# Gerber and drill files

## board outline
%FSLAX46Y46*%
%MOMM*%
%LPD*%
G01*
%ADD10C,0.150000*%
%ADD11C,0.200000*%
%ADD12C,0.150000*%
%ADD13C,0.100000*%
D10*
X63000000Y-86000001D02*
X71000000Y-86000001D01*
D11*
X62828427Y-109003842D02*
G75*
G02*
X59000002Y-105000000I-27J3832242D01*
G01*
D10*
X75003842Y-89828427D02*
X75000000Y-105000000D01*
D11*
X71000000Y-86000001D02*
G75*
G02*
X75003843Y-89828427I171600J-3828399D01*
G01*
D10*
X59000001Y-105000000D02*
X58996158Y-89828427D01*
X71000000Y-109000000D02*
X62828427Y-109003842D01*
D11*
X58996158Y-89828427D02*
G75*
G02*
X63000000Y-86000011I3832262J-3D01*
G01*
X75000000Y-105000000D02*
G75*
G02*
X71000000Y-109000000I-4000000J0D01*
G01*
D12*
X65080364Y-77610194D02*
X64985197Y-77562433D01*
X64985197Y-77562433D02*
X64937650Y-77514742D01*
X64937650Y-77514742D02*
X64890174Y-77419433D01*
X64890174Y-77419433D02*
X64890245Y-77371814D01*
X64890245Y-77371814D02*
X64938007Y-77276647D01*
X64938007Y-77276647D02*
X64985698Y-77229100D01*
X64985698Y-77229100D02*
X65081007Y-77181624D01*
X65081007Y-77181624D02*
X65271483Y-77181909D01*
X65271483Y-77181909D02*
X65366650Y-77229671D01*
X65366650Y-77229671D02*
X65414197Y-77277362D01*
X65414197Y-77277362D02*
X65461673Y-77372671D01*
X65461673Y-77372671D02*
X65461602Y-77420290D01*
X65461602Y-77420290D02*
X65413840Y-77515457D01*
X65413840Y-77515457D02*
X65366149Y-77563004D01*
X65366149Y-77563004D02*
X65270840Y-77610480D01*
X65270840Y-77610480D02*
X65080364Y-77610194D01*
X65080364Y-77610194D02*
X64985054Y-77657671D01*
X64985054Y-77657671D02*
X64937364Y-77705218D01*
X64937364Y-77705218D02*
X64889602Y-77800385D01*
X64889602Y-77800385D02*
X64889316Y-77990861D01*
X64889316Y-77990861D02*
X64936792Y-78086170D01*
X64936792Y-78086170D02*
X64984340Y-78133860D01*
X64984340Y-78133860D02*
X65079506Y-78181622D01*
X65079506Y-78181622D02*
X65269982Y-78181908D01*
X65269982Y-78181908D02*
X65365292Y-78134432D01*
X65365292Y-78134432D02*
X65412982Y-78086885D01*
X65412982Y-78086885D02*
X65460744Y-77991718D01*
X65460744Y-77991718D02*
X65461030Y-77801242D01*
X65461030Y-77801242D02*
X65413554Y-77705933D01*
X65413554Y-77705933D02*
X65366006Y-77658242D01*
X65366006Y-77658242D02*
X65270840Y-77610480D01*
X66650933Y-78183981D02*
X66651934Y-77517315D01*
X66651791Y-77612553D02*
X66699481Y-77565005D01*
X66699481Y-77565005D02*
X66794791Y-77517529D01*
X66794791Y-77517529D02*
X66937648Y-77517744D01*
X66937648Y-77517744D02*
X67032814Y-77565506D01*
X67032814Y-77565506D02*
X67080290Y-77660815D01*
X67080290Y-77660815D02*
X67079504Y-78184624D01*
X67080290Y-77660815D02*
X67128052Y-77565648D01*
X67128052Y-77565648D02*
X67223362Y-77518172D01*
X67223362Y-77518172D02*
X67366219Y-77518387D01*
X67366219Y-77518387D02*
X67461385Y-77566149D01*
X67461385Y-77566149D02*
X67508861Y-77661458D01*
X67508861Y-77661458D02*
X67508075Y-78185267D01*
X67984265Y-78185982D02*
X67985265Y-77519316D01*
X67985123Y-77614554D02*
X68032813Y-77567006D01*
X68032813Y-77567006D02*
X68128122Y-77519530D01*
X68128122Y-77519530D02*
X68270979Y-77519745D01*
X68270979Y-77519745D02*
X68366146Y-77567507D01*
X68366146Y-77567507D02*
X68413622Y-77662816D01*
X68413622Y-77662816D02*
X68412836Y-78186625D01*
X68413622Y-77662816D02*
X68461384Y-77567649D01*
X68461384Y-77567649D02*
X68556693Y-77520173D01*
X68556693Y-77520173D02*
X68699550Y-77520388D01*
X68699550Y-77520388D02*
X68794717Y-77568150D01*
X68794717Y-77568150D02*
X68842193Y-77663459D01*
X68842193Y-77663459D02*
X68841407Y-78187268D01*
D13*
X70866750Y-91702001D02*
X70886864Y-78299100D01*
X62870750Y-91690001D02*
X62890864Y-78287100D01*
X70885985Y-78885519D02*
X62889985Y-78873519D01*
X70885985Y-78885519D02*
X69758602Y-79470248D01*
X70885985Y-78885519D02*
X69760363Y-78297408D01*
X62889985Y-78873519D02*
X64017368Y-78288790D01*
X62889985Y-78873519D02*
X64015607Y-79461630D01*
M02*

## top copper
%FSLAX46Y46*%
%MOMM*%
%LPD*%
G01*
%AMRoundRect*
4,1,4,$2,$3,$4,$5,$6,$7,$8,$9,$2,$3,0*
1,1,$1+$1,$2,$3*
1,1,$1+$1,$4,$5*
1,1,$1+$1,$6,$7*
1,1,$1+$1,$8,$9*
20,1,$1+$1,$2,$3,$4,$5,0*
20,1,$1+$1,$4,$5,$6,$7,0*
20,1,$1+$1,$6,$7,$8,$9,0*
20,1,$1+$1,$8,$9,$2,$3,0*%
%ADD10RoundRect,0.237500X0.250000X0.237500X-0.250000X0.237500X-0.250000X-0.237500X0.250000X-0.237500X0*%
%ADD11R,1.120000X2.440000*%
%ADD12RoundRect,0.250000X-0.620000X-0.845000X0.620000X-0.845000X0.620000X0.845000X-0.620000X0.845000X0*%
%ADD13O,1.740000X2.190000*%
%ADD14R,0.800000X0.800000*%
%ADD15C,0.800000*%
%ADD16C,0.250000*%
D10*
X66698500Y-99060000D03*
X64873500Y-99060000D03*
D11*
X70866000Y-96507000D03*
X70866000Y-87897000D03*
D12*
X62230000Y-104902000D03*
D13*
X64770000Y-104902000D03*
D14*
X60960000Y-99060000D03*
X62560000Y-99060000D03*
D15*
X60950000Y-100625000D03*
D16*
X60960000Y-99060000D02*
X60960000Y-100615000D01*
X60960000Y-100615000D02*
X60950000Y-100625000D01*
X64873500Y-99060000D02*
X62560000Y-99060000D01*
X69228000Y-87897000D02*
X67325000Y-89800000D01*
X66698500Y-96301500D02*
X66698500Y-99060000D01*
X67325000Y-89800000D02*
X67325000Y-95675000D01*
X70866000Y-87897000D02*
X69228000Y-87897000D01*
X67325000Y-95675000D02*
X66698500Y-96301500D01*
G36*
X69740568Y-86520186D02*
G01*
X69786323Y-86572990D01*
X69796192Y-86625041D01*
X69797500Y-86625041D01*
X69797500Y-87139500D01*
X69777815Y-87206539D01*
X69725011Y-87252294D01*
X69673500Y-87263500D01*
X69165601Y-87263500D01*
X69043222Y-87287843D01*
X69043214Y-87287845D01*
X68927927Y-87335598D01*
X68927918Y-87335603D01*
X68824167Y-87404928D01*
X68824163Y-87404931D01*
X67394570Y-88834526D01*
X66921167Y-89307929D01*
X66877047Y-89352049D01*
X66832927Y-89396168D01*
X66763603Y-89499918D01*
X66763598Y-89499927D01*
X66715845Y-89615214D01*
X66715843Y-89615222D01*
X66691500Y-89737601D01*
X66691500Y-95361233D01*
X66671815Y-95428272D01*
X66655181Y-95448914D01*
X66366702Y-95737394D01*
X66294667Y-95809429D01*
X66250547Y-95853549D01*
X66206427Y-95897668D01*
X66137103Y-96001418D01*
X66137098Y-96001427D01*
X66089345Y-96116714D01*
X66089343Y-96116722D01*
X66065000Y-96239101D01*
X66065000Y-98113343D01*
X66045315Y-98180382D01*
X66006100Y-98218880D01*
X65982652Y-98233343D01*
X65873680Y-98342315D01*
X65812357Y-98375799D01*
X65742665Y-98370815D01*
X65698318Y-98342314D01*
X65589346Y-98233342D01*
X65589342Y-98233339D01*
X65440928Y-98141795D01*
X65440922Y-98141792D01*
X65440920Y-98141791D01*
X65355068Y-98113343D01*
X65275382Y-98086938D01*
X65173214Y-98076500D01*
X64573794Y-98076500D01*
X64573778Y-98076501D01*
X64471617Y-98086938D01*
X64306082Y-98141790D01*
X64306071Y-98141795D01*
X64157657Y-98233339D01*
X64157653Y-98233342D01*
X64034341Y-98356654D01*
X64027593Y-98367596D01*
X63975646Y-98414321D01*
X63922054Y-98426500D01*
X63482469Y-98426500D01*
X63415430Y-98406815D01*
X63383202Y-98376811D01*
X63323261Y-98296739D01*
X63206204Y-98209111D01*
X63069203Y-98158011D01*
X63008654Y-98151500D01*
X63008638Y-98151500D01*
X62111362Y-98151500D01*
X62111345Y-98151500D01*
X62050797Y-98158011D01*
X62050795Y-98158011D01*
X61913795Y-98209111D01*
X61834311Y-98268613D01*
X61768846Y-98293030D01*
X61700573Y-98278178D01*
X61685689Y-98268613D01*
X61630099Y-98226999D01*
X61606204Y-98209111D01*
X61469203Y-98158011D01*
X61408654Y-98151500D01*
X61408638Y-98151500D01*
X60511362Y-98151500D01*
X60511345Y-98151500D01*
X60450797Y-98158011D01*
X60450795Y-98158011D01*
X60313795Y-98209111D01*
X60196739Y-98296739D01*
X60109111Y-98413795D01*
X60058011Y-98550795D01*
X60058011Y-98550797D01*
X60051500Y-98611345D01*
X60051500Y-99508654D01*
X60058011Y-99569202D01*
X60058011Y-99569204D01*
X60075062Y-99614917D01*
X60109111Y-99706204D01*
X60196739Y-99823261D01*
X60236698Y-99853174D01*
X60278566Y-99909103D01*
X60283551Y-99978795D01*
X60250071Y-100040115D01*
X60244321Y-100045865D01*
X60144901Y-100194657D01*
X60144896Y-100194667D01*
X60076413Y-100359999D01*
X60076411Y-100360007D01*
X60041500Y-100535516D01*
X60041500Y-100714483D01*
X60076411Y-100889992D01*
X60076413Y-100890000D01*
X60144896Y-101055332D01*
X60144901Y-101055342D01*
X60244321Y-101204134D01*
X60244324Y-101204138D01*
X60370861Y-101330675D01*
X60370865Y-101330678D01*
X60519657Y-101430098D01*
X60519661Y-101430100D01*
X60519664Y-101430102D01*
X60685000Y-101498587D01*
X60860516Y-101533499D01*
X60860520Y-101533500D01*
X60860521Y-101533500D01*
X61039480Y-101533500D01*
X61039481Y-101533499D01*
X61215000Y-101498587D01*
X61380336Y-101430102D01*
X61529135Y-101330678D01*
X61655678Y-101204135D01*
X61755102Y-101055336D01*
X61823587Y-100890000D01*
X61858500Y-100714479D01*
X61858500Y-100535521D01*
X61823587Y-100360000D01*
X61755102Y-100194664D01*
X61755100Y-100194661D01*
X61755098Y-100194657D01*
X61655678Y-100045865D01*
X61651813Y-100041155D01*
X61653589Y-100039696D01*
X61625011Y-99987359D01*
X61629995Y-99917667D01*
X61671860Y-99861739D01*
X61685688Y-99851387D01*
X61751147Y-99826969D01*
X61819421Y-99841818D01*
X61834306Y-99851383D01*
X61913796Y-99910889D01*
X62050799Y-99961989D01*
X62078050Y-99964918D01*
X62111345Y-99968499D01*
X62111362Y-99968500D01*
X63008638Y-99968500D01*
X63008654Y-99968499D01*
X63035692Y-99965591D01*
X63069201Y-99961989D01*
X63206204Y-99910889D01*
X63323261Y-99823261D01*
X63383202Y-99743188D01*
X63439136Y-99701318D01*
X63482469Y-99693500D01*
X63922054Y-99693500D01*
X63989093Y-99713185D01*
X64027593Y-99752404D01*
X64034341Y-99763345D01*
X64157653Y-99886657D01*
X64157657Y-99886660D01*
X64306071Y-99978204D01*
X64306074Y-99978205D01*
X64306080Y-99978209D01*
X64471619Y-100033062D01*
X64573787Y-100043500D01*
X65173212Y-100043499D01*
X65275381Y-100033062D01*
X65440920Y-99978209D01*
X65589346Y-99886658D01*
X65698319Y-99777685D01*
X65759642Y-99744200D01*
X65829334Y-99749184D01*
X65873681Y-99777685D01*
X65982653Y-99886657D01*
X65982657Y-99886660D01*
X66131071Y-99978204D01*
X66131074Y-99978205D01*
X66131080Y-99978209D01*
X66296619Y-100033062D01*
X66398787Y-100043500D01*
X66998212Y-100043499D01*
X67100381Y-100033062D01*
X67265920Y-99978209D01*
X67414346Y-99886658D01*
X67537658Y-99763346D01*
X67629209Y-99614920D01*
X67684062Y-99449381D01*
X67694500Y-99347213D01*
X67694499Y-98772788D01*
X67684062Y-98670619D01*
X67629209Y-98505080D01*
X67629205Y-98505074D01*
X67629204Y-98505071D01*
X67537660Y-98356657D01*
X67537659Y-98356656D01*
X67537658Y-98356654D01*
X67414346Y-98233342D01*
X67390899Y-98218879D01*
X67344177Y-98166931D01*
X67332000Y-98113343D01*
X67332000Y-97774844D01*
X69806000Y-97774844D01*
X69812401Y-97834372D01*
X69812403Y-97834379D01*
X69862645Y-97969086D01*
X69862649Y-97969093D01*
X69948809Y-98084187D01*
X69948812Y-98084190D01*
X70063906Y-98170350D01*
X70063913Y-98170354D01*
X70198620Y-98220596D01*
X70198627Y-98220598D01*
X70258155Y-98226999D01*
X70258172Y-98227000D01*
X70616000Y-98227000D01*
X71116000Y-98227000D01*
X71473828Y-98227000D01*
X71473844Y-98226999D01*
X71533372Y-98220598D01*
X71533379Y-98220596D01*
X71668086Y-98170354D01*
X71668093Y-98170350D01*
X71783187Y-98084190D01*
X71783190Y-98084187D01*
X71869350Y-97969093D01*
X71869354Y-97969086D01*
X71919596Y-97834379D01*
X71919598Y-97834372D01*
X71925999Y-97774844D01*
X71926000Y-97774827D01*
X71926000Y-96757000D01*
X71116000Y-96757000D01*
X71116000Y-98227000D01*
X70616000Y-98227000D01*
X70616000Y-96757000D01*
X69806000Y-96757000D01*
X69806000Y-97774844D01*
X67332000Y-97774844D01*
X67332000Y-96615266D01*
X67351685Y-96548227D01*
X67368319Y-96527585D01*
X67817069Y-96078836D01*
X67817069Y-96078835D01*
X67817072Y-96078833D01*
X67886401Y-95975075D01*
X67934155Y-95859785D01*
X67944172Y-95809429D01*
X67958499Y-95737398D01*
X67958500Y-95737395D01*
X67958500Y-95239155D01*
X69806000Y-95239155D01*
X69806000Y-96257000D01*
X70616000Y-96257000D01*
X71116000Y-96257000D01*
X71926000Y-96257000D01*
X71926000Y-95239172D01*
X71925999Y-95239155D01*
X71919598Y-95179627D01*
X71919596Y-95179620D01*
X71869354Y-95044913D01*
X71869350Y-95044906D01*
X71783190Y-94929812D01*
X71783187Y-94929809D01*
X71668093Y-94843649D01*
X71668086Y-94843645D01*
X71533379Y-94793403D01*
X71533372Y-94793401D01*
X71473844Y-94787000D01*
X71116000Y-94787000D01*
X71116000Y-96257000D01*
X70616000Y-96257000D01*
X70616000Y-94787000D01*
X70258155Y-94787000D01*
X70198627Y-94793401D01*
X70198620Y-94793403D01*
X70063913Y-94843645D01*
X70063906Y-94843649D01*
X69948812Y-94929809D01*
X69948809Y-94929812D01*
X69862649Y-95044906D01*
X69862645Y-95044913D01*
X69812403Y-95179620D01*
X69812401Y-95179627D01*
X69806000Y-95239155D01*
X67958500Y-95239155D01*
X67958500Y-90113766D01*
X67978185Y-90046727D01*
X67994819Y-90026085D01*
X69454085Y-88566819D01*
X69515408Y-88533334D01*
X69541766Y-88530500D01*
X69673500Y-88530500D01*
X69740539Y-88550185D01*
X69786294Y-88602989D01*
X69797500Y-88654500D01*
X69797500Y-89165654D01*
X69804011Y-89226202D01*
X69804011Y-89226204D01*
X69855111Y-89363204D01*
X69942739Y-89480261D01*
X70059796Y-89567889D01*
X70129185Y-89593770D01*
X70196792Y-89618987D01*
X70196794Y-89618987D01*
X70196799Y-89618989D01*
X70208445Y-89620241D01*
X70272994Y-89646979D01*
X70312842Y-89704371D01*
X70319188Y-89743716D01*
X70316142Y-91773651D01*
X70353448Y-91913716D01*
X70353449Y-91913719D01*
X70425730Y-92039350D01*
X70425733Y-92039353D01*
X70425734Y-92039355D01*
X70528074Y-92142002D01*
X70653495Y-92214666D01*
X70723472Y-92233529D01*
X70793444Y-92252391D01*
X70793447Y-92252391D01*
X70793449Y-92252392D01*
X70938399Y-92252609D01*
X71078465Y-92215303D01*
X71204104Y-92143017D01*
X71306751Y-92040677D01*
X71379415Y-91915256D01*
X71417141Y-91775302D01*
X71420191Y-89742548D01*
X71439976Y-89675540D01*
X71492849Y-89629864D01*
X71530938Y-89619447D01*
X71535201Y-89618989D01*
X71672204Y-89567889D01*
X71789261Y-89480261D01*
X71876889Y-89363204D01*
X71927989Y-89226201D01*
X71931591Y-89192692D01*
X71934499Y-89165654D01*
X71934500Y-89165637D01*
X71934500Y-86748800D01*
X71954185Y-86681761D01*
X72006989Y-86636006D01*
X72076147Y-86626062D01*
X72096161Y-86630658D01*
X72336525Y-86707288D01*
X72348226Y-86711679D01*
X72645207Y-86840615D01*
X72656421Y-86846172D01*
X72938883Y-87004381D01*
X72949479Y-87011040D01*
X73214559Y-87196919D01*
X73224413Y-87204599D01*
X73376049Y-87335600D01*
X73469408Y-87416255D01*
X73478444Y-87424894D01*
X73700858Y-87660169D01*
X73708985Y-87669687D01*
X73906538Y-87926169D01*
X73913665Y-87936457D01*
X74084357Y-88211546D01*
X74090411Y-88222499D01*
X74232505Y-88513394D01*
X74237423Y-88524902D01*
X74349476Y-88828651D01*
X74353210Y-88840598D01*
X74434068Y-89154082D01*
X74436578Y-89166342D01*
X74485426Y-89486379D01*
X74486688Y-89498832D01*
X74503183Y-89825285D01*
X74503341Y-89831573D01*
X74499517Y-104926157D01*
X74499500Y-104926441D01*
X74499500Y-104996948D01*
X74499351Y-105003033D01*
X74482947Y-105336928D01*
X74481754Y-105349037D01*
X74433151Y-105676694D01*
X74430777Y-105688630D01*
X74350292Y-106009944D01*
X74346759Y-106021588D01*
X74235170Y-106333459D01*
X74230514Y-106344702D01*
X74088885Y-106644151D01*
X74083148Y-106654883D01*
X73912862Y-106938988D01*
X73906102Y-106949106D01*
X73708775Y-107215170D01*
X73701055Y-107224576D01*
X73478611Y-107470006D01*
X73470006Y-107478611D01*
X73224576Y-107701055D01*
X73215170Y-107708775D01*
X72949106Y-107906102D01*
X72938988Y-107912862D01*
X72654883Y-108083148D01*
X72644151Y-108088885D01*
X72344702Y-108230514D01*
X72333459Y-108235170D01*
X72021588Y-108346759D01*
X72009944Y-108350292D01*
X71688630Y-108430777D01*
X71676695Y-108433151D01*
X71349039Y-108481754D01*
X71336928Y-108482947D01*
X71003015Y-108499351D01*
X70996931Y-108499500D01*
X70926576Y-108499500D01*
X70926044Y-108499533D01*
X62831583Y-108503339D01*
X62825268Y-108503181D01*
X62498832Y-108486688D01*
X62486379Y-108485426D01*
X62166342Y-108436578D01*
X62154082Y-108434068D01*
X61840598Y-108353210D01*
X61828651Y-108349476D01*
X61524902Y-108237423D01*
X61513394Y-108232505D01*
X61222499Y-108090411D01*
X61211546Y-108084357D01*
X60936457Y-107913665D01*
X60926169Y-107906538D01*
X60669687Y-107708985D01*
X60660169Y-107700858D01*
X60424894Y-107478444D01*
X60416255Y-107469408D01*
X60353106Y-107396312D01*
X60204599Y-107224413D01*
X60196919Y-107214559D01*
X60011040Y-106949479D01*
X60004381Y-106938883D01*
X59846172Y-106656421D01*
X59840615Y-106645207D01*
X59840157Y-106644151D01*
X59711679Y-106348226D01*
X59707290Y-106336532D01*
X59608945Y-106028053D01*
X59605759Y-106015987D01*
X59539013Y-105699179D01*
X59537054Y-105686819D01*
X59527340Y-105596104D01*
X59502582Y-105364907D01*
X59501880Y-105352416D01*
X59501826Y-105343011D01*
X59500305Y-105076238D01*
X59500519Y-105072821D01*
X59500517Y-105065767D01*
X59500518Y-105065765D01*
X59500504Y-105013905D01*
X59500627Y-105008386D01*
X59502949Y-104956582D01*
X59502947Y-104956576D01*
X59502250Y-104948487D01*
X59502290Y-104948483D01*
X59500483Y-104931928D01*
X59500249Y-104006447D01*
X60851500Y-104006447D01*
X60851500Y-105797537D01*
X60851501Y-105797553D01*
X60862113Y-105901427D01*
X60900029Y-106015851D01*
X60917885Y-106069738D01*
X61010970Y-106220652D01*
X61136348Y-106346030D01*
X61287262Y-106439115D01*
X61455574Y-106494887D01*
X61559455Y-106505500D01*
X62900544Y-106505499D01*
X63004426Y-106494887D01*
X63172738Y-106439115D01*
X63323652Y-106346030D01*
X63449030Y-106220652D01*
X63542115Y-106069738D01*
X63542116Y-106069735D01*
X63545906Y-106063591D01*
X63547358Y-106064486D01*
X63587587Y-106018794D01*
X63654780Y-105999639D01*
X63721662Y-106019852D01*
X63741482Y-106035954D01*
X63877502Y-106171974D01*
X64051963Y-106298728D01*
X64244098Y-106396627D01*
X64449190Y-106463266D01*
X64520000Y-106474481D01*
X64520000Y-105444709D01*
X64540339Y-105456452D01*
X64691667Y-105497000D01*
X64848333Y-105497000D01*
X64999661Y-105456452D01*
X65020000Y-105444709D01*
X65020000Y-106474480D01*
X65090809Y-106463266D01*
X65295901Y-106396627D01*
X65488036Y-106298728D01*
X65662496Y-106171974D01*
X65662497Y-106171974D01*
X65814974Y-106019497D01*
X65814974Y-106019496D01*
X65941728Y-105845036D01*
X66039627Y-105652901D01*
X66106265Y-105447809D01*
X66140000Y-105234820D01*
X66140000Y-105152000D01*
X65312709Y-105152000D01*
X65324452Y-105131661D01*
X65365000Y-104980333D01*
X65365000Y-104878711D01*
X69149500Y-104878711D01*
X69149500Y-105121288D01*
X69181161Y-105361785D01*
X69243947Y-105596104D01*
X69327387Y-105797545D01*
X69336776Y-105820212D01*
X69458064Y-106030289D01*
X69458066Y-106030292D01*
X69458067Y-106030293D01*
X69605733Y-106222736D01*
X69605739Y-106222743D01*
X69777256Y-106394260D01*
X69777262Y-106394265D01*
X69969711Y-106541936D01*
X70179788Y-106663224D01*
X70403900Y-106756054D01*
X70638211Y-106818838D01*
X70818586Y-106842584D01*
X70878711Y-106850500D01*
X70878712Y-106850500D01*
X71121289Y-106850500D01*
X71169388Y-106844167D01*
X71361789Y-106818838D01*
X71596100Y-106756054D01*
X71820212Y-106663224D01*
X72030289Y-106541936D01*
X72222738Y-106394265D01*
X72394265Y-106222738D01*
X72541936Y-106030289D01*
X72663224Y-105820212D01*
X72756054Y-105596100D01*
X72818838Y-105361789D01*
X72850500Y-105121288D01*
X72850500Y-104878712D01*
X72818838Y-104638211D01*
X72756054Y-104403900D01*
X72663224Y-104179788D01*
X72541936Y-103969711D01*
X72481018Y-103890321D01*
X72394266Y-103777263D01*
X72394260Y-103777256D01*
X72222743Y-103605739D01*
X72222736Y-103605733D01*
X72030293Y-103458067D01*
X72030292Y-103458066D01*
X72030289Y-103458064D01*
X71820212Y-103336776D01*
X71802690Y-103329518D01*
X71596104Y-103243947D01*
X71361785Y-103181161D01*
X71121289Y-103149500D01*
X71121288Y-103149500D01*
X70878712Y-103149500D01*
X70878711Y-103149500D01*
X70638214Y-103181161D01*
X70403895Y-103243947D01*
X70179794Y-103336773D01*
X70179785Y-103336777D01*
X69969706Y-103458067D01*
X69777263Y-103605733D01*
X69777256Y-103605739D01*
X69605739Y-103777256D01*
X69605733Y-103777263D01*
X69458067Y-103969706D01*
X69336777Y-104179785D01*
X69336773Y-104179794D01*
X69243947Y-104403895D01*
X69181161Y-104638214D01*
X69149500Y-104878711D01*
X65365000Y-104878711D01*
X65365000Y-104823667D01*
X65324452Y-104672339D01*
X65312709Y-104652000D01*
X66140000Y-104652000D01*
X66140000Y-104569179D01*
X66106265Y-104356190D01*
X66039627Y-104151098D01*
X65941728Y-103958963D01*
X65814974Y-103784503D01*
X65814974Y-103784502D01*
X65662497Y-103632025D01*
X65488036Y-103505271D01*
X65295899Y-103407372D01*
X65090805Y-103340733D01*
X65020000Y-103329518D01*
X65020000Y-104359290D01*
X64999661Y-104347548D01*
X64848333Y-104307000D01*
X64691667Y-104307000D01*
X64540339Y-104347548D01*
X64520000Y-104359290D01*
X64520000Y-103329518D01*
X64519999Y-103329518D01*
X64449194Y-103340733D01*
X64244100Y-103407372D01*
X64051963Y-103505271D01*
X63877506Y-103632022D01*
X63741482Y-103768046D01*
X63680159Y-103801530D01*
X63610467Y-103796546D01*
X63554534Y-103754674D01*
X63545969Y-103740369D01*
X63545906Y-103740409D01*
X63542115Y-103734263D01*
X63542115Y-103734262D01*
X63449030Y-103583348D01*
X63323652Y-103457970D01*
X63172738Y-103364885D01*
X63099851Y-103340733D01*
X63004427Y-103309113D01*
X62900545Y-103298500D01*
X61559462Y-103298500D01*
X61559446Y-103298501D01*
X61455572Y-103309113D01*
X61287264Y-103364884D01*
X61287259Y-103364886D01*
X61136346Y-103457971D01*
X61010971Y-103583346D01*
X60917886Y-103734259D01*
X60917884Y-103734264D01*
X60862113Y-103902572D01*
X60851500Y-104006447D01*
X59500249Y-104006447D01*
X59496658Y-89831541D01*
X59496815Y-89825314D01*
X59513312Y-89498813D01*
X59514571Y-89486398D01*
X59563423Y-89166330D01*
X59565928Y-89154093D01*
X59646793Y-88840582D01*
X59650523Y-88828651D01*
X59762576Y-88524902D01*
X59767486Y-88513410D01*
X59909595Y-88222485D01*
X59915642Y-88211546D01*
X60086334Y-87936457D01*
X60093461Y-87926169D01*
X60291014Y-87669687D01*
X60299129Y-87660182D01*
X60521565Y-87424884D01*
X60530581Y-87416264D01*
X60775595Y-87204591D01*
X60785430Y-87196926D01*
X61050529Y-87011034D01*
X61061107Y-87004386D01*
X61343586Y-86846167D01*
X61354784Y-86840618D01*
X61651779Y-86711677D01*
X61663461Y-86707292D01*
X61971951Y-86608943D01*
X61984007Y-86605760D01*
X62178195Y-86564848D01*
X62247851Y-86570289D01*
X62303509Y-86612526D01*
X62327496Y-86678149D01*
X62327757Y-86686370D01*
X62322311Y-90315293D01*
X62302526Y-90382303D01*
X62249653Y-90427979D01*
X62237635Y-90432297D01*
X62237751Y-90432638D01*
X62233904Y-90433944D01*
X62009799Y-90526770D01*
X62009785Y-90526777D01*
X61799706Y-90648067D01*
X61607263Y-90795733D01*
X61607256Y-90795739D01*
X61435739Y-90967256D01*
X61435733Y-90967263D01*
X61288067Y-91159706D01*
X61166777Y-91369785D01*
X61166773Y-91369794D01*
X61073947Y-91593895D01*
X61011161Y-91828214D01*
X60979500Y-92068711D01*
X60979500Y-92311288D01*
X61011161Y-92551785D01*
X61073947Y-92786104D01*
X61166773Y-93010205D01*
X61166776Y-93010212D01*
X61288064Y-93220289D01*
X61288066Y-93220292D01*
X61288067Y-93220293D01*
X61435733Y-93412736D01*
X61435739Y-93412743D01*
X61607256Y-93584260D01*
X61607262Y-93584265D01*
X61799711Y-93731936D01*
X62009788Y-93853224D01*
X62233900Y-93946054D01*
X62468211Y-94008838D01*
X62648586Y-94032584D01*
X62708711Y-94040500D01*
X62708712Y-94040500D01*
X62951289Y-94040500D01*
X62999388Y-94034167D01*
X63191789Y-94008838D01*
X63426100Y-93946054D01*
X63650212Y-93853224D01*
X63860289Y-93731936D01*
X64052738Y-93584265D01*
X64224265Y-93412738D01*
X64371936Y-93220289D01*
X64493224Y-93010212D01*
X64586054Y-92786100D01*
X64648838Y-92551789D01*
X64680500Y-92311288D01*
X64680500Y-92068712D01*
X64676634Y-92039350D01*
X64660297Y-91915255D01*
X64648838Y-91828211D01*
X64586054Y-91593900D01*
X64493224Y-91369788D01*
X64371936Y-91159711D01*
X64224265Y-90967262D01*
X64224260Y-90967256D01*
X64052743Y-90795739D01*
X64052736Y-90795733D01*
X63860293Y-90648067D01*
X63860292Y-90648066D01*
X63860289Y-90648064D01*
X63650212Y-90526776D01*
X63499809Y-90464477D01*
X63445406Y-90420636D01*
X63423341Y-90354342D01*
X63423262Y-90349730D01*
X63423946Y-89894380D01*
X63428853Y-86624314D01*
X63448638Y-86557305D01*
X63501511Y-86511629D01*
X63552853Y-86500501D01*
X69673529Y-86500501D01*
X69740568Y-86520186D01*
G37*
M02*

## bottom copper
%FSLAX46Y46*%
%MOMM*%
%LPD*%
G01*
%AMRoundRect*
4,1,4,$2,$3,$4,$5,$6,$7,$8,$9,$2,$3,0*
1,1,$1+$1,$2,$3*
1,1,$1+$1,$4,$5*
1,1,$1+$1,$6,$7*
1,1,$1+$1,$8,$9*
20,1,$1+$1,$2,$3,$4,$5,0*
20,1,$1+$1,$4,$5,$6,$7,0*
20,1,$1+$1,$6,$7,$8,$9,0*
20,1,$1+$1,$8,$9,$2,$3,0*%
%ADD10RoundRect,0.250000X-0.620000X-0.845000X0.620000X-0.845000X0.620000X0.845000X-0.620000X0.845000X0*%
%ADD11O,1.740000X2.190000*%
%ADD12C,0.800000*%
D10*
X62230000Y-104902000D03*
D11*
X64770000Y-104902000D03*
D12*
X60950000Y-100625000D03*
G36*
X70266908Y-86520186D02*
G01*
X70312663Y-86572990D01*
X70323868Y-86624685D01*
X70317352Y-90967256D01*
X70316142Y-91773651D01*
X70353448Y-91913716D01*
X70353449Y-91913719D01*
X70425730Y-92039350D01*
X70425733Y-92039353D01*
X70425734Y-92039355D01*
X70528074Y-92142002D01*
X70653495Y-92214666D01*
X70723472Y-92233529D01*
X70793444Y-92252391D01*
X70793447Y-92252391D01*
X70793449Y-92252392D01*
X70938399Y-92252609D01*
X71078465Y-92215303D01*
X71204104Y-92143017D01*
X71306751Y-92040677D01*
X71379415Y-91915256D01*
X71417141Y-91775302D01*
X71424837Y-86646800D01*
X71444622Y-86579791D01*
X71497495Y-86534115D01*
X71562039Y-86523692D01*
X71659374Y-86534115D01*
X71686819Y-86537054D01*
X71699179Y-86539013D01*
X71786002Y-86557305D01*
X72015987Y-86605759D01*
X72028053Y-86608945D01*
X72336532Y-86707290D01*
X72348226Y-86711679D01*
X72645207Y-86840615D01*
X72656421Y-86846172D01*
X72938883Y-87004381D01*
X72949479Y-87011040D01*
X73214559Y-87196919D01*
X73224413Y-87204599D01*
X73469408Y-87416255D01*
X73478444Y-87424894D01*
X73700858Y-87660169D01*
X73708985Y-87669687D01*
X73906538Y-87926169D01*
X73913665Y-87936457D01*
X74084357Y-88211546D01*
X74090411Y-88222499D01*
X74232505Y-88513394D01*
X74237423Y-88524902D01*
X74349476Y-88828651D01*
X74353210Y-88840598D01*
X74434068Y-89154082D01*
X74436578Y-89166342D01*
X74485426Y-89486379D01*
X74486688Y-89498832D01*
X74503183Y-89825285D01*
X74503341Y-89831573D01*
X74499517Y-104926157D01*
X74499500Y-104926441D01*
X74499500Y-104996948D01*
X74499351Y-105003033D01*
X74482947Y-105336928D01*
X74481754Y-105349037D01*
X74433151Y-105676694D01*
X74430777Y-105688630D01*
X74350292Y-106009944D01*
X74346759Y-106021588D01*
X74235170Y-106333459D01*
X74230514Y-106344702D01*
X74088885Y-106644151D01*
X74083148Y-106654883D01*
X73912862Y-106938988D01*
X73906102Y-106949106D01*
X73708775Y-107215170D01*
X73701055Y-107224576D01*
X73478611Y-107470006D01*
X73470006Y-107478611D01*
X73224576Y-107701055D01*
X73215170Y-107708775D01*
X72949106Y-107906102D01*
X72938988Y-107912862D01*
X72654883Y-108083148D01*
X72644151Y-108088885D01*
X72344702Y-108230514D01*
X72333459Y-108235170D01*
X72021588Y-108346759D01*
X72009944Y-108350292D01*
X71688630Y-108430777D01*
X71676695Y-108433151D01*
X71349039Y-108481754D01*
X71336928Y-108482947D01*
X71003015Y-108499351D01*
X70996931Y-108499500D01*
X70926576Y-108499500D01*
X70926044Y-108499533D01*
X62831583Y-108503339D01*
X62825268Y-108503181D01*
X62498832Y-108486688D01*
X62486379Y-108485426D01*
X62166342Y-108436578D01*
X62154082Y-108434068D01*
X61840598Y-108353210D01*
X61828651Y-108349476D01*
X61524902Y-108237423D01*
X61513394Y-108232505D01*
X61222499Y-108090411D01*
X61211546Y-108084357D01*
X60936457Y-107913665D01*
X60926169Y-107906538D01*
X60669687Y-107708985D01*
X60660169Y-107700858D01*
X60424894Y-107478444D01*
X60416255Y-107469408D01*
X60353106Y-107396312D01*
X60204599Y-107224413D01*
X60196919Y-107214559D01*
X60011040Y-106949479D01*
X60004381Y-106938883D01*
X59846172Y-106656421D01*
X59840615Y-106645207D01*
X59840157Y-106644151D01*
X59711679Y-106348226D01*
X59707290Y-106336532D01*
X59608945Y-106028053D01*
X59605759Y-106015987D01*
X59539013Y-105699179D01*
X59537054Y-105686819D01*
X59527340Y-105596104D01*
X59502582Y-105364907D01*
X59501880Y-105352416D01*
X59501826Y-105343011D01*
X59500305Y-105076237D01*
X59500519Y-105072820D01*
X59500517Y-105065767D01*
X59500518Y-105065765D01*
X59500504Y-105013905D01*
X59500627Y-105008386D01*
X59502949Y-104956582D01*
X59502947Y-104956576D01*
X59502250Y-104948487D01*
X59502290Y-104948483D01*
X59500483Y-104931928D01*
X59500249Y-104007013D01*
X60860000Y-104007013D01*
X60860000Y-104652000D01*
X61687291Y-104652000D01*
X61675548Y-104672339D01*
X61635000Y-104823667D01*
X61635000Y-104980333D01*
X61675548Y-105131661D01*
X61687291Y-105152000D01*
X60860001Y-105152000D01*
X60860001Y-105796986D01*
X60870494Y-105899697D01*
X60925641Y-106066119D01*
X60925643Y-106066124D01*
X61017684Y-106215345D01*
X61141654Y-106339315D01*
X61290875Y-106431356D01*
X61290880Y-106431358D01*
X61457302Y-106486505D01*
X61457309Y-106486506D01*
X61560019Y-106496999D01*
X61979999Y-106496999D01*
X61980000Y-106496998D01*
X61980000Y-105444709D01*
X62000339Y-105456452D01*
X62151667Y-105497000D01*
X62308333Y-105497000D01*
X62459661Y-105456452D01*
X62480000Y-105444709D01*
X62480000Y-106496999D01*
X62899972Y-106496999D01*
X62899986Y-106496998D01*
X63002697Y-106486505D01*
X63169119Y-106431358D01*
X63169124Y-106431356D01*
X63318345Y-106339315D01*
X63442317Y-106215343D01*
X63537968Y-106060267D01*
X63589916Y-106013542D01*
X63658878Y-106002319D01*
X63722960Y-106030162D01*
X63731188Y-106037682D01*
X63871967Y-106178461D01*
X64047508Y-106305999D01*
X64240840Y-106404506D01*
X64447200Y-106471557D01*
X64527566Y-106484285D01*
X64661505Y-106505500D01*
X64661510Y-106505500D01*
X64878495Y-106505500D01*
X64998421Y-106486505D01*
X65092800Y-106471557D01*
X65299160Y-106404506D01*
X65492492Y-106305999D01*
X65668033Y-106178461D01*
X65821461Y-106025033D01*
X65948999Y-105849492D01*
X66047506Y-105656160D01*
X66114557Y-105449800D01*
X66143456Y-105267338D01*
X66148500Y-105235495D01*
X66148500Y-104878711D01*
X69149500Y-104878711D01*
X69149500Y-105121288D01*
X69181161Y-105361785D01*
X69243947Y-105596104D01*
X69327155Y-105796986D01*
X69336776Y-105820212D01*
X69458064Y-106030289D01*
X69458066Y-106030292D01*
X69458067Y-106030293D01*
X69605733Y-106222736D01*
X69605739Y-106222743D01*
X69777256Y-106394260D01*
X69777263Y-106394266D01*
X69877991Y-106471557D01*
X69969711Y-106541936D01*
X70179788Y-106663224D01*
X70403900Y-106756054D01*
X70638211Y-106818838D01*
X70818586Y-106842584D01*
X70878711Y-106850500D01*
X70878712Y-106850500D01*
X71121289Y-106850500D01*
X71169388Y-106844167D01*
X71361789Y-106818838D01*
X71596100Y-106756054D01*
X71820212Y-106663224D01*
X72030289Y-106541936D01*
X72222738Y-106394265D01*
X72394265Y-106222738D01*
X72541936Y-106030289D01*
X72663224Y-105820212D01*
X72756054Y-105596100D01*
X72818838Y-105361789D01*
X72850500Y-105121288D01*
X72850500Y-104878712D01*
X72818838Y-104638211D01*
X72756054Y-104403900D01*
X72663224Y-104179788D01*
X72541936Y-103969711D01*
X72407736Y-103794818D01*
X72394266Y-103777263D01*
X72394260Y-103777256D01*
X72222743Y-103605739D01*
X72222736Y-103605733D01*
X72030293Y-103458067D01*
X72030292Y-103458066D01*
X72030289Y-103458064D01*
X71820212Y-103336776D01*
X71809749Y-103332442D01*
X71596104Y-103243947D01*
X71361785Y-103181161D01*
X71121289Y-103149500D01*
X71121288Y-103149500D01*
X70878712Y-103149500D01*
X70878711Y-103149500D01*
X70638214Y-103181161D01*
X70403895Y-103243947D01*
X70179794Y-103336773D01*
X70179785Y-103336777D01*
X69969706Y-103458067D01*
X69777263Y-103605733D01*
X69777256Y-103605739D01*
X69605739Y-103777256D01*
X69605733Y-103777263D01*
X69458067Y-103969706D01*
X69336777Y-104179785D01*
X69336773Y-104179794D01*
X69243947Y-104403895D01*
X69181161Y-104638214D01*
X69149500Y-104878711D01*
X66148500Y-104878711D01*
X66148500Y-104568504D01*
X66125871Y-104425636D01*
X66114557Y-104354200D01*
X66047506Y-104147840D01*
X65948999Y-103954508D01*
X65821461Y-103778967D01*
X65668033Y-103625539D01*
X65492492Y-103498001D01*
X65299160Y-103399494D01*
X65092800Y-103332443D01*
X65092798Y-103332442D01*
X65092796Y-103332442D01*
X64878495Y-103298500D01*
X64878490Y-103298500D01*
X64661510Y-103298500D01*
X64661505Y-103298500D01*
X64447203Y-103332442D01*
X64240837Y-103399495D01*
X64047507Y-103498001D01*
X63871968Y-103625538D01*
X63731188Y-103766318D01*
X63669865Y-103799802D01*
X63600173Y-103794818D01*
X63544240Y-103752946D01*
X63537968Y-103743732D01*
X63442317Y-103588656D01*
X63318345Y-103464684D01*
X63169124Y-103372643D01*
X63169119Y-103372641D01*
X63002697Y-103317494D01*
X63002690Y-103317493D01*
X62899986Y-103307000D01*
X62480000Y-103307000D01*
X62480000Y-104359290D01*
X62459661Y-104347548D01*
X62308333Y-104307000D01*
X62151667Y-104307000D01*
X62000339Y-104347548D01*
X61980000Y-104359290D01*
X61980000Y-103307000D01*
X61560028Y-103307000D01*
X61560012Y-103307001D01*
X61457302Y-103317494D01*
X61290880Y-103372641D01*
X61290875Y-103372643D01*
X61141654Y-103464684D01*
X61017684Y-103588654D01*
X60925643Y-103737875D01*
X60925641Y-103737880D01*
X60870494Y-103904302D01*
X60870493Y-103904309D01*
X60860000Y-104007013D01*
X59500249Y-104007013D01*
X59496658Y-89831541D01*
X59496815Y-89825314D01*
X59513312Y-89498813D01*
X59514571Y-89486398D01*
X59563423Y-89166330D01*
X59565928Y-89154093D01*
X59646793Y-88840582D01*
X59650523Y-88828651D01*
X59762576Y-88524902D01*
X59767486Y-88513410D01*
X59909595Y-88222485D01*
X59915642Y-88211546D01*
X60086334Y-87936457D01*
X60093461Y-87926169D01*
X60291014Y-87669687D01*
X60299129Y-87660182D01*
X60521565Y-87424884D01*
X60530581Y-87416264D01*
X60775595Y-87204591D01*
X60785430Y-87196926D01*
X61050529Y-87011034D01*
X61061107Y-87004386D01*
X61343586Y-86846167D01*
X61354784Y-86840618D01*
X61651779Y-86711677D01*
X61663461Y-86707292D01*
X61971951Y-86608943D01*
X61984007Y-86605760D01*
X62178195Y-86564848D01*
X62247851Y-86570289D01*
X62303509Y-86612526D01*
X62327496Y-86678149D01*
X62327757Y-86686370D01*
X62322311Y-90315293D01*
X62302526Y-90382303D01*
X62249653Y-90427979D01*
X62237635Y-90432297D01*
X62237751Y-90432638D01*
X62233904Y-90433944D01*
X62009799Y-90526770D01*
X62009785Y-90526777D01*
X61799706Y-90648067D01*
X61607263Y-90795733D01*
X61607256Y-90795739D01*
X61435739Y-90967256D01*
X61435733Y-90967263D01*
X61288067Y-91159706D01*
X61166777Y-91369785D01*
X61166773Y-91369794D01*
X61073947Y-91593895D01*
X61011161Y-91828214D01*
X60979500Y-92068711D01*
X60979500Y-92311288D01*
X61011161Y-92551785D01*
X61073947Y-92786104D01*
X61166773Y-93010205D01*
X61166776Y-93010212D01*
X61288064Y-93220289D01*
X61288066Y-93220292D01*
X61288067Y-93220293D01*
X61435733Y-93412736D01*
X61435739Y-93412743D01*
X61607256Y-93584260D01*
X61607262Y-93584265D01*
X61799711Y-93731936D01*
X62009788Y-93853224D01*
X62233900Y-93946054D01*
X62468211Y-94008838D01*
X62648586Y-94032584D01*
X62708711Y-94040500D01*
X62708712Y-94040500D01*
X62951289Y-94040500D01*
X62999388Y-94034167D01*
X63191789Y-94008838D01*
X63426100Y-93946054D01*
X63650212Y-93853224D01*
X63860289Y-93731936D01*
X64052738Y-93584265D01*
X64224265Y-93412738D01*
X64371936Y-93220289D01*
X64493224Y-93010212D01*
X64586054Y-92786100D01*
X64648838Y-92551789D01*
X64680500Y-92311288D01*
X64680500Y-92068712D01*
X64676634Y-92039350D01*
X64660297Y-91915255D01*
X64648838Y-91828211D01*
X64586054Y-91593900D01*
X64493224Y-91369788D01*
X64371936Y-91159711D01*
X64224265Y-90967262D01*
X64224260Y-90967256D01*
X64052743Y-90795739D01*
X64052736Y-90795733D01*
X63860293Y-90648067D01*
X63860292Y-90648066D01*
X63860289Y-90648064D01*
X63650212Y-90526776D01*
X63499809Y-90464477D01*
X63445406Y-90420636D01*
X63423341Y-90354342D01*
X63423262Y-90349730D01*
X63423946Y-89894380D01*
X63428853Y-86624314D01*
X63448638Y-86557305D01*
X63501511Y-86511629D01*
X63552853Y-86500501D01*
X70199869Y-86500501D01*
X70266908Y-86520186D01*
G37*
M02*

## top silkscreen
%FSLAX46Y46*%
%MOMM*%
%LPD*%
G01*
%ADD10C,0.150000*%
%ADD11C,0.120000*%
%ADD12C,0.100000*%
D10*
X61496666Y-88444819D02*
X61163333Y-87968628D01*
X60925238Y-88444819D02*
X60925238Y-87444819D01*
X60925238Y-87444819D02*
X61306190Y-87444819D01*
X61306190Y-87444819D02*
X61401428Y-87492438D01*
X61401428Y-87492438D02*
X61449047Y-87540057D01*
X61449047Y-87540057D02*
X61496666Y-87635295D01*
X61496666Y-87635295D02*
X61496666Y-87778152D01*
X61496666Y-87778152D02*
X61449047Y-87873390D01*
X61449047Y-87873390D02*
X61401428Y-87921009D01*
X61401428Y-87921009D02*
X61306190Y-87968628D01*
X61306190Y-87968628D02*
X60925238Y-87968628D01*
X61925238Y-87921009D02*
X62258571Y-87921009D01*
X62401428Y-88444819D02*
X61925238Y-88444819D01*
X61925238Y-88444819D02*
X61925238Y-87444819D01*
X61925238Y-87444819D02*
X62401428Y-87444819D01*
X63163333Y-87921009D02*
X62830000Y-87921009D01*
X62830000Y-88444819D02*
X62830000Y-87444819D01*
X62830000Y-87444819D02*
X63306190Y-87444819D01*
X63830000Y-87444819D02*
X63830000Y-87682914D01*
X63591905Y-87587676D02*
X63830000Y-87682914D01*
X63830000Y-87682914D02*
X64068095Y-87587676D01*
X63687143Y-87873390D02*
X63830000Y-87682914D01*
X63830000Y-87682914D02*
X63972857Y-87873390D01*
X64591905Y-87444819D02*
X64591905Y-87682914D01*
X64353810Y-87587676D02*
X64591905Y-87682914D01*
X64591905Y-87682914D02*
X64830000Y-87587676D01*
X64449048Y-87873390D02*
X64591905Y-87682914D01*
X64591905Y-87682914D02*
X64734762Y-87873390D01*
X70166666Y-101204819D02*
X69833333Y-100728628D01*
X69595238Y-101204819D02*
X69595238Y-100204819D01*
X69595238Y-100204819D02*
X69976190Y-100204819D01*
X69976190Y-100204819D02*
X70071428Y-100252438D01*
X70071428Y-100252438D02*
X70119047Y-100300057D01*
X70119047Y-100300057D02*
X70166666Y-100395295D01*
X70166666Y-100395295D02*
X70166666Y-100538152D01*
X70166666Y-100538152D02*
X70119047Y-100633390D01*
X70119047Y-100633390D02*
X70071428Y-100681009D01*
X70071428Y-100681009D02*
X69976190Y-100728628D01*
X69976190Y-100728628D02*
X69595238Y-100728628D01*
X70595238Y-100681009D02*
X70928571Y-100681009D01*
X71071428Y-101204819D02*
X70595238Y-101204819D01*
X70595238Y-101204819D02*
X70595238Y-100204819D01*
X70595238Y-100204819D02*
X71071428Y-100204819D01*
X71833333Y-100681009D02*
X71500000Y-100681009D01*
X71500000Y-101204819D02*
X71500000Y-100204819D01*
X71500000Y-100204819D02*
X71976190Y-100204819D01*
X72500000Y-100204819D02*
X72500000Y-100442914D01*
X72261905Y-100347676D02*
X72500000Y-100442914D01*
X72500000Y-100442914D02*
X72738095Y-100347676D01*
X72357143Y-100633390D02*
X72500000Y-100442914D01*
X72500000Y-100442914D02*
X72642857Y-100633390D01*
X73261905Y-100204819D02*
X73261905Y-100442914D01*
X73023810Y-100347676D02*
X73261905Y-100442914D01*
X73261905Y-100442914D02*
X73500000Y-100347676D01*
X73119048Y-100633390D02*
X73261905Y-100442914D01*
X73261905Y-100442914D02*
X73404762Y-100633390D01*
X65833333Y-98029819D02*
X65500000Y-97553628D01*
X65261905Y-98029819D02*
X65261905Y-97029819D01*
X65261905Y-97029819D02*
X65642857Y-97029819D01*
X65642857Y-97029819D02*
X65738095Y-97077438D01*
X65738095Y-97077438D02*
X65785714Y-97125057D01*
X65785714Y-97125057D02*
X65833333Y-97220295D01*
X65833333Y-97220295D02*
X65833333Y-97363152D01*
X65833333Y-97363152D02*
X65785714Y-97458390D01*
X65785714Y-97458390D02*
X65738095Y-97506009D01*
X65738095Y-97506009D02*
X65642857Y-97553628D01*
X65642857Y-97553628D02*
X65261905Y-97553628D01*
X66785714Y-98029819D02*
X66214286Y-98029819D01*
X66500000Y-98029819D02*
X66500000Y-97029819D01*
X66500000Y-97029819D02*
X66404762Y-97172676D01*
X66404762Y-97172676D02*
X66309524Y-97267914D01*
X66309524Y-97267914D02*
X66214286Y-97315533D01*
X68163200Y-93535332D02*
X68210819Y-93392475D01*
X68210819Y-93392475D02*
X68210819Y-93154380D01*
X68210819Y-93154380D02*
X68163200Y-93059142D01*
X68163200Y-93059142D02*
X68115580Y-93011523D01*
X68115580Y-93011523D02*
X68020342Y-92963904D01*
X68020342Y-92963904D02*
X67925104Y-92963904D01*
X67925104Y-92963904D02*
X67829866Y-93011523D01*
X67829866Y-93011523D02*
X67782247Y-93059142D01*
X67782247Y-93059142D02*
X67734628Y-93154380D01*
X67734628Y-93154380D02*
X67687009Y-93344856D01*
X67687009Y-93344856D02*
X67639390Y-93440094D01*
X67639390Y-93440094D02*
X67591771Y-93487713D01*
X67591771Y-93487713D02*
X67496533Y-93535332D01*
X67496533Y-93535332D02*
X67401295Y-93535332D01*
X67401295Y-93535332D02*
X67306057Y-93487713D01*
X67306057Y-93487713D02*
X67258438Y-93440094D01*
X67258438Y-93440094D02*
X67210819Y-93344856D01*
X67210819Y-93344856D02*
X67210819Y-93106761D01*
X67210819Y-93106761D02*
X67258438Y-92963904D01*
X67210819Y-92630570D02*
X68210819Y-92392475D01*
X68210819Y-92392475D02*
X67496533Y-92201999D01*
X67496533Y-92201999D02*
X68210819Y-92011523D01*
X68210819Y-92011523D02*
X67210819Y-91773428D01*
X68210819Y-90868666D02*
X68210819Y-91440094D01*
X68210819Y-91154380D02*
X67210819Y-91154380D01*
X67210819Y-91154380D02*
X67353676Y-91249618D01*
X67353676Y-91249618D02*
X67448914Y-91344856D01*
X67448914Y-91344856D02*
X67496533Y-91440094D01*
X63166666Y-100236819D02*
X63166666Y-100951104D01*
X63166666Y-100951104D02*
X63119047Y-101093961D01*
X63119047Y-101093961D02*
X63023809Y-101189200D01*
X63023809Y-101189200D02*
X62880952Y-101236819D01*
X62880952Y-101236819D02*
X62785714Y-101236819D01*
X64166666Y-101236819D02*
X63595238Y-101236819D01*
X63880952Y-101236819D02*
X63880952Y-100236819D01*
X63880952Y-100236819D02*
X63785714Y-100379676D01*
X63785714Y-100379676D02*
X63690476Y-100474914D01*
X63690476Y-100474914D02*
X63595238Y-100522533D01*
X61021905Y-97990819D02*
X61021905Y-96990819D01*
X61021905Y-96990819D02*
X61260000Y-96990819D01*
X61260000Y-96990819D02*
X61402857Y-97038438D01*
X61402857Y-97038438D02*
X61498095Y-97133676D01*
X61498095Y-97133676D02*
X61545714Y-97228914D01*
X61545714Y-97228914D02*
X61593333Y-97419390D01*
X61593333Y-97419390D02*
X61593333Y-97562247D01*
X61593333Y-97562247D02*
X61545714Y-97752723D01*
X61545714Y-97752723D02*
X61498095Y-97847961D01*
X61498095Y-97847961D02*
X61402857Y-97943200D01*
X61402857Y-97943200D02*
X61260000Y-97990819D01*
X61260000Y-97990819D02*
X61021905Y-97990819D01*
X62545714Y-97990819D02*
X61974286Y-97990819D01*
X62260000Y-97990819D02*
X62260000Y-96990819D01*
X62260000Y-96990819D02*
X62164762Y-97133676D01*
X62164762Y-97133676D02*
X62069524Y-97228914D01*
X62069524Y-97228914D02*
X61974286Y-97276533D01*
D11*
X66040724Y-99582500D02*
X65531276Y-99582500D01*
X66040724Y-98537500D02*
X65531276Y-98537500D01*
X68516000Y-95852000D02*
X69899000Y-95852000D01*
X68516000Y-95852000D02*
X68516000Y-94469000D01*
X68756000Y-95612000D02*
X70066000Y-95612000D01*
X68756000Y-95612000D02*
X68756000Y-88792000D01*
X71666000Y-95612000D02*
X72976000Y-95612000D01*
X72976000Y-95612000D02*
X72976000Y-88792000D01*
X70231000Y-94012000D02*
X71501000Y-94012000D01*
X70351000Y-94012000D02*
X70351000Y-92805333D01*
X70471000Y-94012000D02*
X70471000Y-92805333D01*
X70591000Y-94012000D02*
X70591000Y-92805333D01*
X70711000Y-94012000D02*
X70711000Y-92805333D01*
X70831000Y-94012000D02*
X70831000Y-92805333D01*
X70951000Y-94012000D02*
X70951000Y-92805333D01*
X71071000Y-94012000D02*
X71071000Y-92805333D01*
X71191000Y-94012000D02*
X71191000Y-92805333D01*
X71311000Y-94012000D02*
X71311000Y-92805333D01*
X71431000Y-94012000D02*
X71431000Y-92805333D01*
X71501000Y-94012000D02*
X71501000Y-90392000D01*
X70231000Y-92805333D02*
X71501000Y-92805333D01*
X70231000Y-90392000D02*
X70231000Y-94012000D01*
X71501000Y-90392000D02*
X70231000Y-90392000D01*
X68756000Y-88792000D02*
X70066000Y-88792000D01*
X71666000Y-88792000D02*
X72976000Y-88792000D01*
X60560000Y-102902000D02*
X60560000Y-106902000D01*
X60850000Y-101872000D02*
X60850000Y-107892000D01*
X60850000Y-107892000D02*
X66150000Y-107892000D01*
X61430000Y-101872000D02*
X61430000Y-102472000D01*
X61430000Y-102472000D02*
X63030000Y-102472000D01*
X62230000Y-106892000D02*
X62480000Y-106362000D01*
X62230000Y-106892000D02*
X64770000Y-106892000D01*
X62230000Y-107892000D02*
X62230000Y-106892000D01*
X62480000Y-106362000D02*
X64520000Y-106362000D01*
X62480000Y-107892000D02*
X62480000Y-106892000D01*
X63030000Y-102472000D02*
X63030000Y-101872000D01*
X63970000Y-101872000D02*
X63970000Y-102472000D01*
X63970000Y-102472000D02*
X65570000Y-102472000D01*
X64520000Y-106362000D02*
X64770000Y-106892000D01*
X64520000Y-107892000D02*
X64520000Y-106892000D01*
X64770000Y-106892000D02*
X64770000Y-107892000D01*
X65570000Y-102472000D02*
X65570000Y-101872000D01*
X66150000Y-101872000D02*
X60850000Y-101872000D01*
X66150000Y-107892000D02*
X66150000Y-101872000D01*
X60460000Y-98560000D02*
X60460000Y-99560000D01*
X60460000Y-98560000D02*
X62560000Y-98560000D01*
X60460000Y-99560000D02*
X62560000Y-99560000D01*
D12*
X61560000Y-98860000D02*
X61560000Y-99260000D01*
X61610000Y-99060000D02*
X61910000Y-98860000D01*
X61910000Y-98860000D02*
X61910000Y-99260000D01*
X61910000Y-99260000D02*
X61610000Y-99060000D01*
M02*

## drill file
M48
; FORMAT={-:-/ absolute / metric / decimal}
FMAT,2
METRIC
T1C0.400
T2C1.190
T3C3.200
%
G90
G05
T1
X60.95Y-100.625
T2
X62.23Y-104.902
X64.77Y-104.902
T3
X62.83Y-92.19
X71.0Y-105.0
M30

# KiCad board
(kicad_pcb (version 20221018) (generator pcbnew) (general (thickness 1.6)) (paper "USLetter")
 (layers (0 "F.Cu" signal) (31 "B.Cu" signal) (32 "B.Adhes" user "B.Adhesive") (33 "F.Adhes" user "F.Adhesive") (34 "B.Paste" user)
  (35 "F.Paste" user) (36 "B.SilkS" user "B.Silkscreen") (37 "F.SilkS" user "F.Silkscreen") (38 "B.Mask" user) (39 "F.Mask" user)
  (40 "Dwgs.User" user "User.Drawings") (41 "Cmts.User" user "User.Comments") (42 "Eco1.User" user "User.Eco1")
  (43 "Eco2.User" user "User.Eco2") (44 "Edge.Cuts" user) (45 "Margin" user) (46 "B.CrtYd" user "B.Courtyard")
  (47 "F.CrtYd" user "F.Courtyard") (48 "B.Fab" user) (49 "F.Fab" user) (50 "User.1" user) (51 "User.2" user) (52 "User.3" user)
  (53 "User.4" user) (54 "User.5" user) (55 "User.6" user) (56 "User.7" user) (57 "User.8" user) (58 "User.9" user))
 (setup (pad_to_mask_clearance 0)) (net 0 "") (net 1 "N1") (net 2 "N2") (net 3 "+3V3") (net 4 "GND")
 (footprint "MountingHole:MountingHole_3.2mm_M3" (layer "F.Cu") (at 62.83 92.19)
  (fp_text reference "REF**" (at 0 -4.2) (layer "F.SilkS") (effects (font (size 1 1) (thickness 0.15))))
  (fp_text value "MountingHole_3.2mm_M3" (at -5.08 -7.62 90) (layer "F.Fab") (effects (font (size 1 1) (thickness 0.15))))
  (pad "" np_thru_hole circle (at 0 0) (size 3.2 3.2) (drill 3.2) (layers "*.Cu" "*.Mask")))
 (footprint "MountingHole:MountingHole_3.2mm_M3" (layer "F.Cu") (at 71 105)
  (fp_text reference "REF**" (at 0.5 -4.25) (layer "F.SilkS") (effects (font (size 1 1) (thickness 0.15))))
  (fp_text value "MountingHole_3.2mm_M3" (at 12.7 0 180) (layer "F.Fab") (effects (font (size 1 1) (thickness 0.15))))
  (pad "" np_thru_hole circle (at 0 0) (size 3.2 3.2) (drill 3.2) (layers "*.Cu" "*.Mask")))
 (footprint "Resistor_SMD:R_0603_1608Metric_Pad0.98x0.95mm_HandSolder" (layer "F.Cu") (at 65.786 99.06 180)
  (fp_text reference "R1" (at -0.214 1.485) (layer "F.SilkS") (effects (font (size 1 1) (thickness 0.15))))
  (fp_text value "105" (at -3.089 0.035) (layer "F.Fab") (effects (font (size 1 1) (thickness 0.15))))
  (fp_line (start -0.254724 -0.5225) (end 0.254724 -0.5225) (stroke (width 0.12) (type solid)) (layer "F.SilkS"))
  (fp_line (start -0.254724 0.5225) (end 0.254724 0.5225) (stroke (width 0.12) (type solid)) (layer "F.SilkS"))
  (pad "1" smd roundrect (at -0.9125 0 180) (size 0.975 0.95) (layers "F.Cu" "F.Paste" "F.Mask") (roundrect_rratio 0.25) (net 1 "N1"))
  (pad "2" smd roundrect (at 0.9125 0 180) (size 0.975 0.95) (layers "F.Cu" "F.Paste" "F.Mask") (roundrect_rratio 0.25) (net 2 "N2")))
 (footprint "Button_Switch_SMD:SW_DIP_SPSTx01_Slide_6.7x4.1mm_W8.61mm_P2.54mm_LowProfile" (layer "F.Cu") (at 70.866 92.202 90)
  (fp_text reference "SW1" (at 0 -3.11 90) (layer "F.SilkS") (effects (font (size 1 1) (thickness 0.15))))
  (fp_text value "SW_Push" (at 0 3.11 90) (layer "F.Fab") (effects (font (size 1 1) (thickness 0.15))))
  (fp_line (start -3.65 -2.35) (end -3.65 -0.967) (stroke (width 0.12) (type solid)) (layer "F.SilkS"))
  (fp_line (start -3.65 -2.35) (end -2.267 -2.35) (stroke (width 0.12) (type solid)) (layer "F.SilkS"))
  (fp_line (start -3.41 -2.11) (end -3.41 -0.8) (stroke (width 0.12) (type solid)) (layer "F.SilkS"))
  (fp_line (start -3.41 -2.11) (end 3.41 -2.11) (stroke (width 0.12) (type solid)) (layer "F.SilkS"))
  (fp_line (start -3.41 0.8) (end -3.41 2.11) (stroke (width 0.12) (type solid)) (layer "F.SilkS"))
  (fp_line (start -3.41 2.11) (end 3.41 2.11) (stroke (width 0.12) (type solid)) (layer "F.SilkS"))
  (fp_line (start -1.81 -0.635) (end -1.81 0.635) (stroke (width 0.12) (type solid)) (layer "F.SilkS"))
  (fp_line (start -1.81 -0.515) (end -0.603333 -0.515) (stroke (width 0.12) (type solid)) (layer "F.SilkS"))
  (fp_line (start -1.81 -0.395) (end -0.603333 -0.395) (stroke (width 0.12) (type solid)) (layer "F.SilkS"))
  (fp_line (start -1.81 -0.275) (end -0.603333 -0.275) (stroke (width 0.12) (type solid)) (layer "F.SilkS"))
  (fp_line (start -1.81 -0.155) (end -0.603333 -0.155) (stroke (width 0.12) (type solid)) (layer "F.SilkS"))
  (fp_line (start -1.81 -0.035) (end -0.603333 -0.035) (stroke (width 0.12) (type solid)) (layer "F.SilkS"))
  (fp_line (start -1.81 0.085) (end -0.603333 0.085) (stroke (width 0.12) (type solid)) (layer "F.SilkS"))
  (fp_line (start -1.81 0.205) (end -0.603333 0.205) (stroke (width 0.12) (type solid)) (layer "F.SilkS"))
  (fp_line (start -1.81 0.325) (end -0.603333 0.325) (stroke (width 0.12) (type solid)) (layer "F.SilkS"))
  (fp_line (start -1.81 0.445) (end -0.603333 0.445) (stroke (width 0.12) (type solid)) (layer "F.SilkS"))
  (fp_line (start -1.81 0.565) (end -0.603333 0.565) (stroke (width 0.12) (type solid)) (layer "F.SilkS"))
  (fp_line (start -1.81 0.635) (end 1.81 0.635) (stroke (width 0.12) (type solid)) (layer "F.SilkS"))
  (fp_line (start -0.603333 -0.635) (end -0.603333 0.635) (stroke (width 0.12) (type solid)) (layer "F.SilkS"))
  (fp_line (start 1.81 -0.635) (end -1.81 -0.635) (stroke (width 0.12) (type solid)) (layer "F.SilkS"))
  (fp_line (start 1.81 0.635) (end 1.81 -0.635) (stroke (width 0.12) (type solid)) (layer "F.SilkS"))
  (fp_line (start 3.41 -2.11) (end 3.41 -0.8) (stroke (width 0.12) (type solid)) (layer "F.SilkS"))
  (fp_line (start 3.41 0.8) (end 3.41 2.11) (stroke (width 0.12) (type solid)) (layer "F.SilkS"))
  (pad "1" smd rect (at -4.305 0 90) (size 2.44 1.12) (layers "F.Cu" "F.Paste" "F.Mask") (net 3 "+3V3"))
  (pad "2" smd rect (at 4.305 0 90) (size 2.44 1.12) (layers "F.Cu" "F.Paste" "F.Mask") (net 1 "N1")))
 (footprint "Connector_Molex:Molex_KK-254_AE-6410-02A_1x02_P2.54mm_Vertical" (layer "F.Cu") (at 62.23 104.902)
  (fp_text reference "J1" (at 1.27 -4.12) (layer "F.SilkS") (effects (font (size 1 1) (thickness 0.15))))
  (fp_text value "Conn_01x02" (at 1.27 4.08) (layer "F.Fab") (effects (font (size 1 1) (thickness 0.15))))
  (fp_line (start -1.67 -2) (end -1.67 2) (stroke (width 0.12) (type solid)) (layer "F.SilkS"))
  (fp_line (start -1.38 -3.03) (end -1.38 2.99) (stroke (width 0.12) (type solid)) (layer "F.SilkS"))
  (fp_line (start -1.38 2.99) (end 3.92 2.99) (stroke (width 0.12) (type solid)) (layer "F.SilkS"))
  (fp_line (start -0.8 -3.03) (end -0.8 -2.43) (stroke (width 0.12) (type solid)) (layer "F.SilkS"))
  (fp_line (start -0.8 -2.43) (end 0.8 -2.43) (stroke (width 0.12) (type solid)) (layer "F.SilkS"))
  (fp_line (start 0 1.99) (end 0.25 1.46) (stroke (width 0.12) (type solid)) (layer "F.SilkS"))
  (fp_line (start 0 1.99) (end 2.54 1.99) (stroke (width 0.12) (type solid)) (layer "F.SilkS"))
  (fp_line (start 0 2.99) (end 0 1.99) (stroke (width 0.12) (type solid)) (layer "F.SilkS"))
  (fp_line (start 0.25 1.46) (end 2.29 1.46) (stroke (width 0.12) (type solid)) (layer "F.SilkS"))
  (fp_line (start 0.25 2.99) (end 0.25 1.99) (stroke (width 0.12) (type solid)) (layer "F.SilkS"))
  (fp_line (start 0.8 -2.43) (end 0.8 -3.03) (stroke (width 0.12) (type solid)) (layer "F.SilkS"))
  (fp_line (start 1.74 -3.03) (end 1.74 -2.43) (stroke (width 0.12) (type solid)) (layer "F.SilkS"))
  (fp_line (start 1.74 -2.43) (end 3.34 -2.43) (stroke (width 0.12) (type solid)) (layer "F.SilkS"))
  (fp_line (start 2.29 1.46) (end 2.54 1.99) (stroke (width 0.12) (type solid)) (layer "F.SilkS"))
  (fp_line (start 2.29 2.99) (end 2.29 1.99) (stroke (width 0.12) (type solid)) (layer "F.SilkS"))
  (fp_line (start 2.54 1.99) (end 2.54 2.99) (stroke (width 0.12) (type solid)) (layer "F.SilkS"))
  (fp_line (start 3.34 -2.43) (end 3.34 -3.03) (stroke (width 0.12) (type solid)) (layer "F.SilkS"))
  (fp_line (start 3.92 -3.03) (end -1.38 -3.03) (stroke (width 0.12) (type solid)) (layer "F.SilkS"))
  (fp_line (start 3.92 2.99) (end 3.92 -3.03) (stroke (width 0.12) (type solid)) (layer "F.SilkS"))
  (pad "1" thru_hole roundrect (at 0 0) (size 1.74 2.19) (drill 1.19) (layers "*.Cu" "*.Mask") (roundrect_rratio 0.143678) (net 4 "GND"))
  (pad "2" thru_hole oval (at 2.54 0) (size 1.74 2.19) (drill 1.19) (layers "*.Cu" "*.Mask") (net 3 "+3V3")))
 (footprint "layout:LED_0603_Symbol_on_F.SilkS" (layer "F.Cu") (at 61.76 99.06)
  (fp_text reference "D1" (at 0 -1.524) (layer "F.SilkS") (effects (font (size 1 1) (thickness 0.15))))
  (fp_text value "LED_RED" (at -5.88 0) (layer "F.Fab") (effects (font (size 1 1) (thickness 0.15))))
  (fp_line (start -1.3 -0.5) (end -1.3 0.5) (stroke (width 0.12) (type solid)) (layer "F.SilkS"))
  (fp_line (start -1.3 -0.5) (end 0.8 -0.5) (stroke (width 0.12) (type solid)) (layer "F.SilkS"))
  (fp_line (start -1.3 0.5) (end 0.8 0.5) (stroke (width 0.12) (type solid)) (layer "F.SilkS"))
  (fp_line (start -0.2 -0.2) (end -0.2 0.2) (stroke (width 0.1) (type solid)) (layer "F.SilkS"))
  (fp_line (start -0.15 0) (end 0.15 -0.2) (stroke (width 0.1) (type solid)) (layer "F.SilkS"))
  (fp_line (start 0.15 -0.2) (end 0.15 0.2) (stroke (width 0.1) (type solid)) (layer "F.SilkS"))
  (fp_line (start 0.15 0.2) (end -0.15 0) (stroke (width 0.1) (type solid)) (layer "F.SilkS"))
  (pad "1" smd rect (at -0.8 0 180) (size 0.8 0.8) (layers "F.Cu" "F.Paste" "F.Mask") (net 4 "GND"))
  (pad "2" smd rect (at 0.8 0 180) (size 0.8 0.8) (layers "F.Cu" "F.Paste" "F.Mask") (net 2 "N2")))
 (gr_line (start 63 86.000001) (end 71 86.000001) (stroke (width 0.15) (type default)) (layer "Edge.Cuts"))
 (gr_arc (start 62.828427 109.003842) (mid 60.058607 107.820042) (end 59.000001 105) (stroke (width 0.2) (type default)) (layer "Edge.Cuts"))
 (gr_line (start 75.003842 89.828427) (end 75 105) (stroke (width 0.15) (type default)) (layer "Edge.Cuts"))
 (gr_arc (start 71 86.000001) (mid 73.820042 87.058607) (end 75.003842 89.828427) (stroke (width 0.2) (type default)) (layer "Edge.Cuts"))
 (gr_line (start 59.000001 105) (end 58.996158 89.828427) (stroke (width 0.15) (type default)) (layer "Edge.Cuts"))
 (gr_line (start 71 109) (end 62.828427 109.003842) (stroke (width 0.15) (type default)) (layer "Edge.Cuts"))
 (gr_arc (start 58.996158 89.828427) (mid 60.179958 87.058607) (end 63 86.000001) (stroke (width 0.2) (type default)) (layer "Edge.Cuts"))
 (gr_arc (start 75 105) (mid 73.828427 107.828427) (end 71 109) (stroke (width 0.2) (type default)) (layer "Edge.Cuts"))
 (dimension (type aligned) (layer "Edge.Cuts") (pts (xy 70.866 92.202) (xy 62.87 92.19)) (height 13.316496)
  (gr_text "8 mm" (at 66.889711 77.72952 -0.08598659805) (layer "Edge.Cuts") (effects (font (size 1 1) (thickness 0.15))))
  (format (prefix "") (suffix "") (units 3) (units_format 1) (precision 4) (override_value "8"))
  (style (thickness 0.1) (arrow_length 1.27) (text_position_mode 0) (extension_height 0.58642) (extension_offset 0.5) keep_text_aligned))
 (segment (start 60.96 99.06) (end 60.96 100.615) (width 0.25) (layer "F.Cu") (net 4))
 (segment (start 60.96 100.615) (end 60.95 100.625) (width 0.25) (layer "F.Cu") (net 4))
 (via (at 60.95 100.625) (size 0.8) (drill 0.4) (layers "F.Cu" "B.Cu") (free) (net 4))
 (segment (start 64.8735 99.06) (end 62.56 99.06) (width 0.25) (layer "F.Cu") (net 2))
 (segment (start 69.228 87.897) (end 67.325 89.8) (width 0.25) (layer "F.Cu") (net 1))
 (segment (start 66.6985 96.3015) (end 66.6985 99.06) (width 0.25) (layer "F.Cu") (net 1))
 (segment (start 67.325 89.8) (end 67.325 95.675) (width 0.25) (layer "F.Cu") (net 1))
 (segment (start 70.866 87.897) (end 69.228 87.897) (width 0.25) (layer "F.Cu") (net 1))
 (segment (start 67.325 95.675) (end 66.6985 96.3015) (width 0.25) (layer "F.Cu") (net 1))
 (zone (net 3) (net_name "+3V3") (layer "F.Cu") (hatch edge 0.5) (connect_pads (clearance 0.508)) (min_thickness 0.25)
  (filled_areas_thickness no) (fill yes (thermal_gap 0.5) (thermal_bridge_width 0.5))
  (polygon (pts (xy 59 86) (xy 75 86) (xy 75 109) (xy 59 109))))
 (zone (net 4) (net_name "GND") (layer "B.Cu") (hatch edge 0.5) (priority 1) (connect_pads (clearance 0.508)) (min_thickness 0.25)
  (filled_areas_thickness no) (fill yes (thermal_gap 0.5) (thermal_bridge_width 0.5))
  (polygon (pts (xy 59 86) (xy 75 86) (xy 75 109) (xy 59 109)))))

